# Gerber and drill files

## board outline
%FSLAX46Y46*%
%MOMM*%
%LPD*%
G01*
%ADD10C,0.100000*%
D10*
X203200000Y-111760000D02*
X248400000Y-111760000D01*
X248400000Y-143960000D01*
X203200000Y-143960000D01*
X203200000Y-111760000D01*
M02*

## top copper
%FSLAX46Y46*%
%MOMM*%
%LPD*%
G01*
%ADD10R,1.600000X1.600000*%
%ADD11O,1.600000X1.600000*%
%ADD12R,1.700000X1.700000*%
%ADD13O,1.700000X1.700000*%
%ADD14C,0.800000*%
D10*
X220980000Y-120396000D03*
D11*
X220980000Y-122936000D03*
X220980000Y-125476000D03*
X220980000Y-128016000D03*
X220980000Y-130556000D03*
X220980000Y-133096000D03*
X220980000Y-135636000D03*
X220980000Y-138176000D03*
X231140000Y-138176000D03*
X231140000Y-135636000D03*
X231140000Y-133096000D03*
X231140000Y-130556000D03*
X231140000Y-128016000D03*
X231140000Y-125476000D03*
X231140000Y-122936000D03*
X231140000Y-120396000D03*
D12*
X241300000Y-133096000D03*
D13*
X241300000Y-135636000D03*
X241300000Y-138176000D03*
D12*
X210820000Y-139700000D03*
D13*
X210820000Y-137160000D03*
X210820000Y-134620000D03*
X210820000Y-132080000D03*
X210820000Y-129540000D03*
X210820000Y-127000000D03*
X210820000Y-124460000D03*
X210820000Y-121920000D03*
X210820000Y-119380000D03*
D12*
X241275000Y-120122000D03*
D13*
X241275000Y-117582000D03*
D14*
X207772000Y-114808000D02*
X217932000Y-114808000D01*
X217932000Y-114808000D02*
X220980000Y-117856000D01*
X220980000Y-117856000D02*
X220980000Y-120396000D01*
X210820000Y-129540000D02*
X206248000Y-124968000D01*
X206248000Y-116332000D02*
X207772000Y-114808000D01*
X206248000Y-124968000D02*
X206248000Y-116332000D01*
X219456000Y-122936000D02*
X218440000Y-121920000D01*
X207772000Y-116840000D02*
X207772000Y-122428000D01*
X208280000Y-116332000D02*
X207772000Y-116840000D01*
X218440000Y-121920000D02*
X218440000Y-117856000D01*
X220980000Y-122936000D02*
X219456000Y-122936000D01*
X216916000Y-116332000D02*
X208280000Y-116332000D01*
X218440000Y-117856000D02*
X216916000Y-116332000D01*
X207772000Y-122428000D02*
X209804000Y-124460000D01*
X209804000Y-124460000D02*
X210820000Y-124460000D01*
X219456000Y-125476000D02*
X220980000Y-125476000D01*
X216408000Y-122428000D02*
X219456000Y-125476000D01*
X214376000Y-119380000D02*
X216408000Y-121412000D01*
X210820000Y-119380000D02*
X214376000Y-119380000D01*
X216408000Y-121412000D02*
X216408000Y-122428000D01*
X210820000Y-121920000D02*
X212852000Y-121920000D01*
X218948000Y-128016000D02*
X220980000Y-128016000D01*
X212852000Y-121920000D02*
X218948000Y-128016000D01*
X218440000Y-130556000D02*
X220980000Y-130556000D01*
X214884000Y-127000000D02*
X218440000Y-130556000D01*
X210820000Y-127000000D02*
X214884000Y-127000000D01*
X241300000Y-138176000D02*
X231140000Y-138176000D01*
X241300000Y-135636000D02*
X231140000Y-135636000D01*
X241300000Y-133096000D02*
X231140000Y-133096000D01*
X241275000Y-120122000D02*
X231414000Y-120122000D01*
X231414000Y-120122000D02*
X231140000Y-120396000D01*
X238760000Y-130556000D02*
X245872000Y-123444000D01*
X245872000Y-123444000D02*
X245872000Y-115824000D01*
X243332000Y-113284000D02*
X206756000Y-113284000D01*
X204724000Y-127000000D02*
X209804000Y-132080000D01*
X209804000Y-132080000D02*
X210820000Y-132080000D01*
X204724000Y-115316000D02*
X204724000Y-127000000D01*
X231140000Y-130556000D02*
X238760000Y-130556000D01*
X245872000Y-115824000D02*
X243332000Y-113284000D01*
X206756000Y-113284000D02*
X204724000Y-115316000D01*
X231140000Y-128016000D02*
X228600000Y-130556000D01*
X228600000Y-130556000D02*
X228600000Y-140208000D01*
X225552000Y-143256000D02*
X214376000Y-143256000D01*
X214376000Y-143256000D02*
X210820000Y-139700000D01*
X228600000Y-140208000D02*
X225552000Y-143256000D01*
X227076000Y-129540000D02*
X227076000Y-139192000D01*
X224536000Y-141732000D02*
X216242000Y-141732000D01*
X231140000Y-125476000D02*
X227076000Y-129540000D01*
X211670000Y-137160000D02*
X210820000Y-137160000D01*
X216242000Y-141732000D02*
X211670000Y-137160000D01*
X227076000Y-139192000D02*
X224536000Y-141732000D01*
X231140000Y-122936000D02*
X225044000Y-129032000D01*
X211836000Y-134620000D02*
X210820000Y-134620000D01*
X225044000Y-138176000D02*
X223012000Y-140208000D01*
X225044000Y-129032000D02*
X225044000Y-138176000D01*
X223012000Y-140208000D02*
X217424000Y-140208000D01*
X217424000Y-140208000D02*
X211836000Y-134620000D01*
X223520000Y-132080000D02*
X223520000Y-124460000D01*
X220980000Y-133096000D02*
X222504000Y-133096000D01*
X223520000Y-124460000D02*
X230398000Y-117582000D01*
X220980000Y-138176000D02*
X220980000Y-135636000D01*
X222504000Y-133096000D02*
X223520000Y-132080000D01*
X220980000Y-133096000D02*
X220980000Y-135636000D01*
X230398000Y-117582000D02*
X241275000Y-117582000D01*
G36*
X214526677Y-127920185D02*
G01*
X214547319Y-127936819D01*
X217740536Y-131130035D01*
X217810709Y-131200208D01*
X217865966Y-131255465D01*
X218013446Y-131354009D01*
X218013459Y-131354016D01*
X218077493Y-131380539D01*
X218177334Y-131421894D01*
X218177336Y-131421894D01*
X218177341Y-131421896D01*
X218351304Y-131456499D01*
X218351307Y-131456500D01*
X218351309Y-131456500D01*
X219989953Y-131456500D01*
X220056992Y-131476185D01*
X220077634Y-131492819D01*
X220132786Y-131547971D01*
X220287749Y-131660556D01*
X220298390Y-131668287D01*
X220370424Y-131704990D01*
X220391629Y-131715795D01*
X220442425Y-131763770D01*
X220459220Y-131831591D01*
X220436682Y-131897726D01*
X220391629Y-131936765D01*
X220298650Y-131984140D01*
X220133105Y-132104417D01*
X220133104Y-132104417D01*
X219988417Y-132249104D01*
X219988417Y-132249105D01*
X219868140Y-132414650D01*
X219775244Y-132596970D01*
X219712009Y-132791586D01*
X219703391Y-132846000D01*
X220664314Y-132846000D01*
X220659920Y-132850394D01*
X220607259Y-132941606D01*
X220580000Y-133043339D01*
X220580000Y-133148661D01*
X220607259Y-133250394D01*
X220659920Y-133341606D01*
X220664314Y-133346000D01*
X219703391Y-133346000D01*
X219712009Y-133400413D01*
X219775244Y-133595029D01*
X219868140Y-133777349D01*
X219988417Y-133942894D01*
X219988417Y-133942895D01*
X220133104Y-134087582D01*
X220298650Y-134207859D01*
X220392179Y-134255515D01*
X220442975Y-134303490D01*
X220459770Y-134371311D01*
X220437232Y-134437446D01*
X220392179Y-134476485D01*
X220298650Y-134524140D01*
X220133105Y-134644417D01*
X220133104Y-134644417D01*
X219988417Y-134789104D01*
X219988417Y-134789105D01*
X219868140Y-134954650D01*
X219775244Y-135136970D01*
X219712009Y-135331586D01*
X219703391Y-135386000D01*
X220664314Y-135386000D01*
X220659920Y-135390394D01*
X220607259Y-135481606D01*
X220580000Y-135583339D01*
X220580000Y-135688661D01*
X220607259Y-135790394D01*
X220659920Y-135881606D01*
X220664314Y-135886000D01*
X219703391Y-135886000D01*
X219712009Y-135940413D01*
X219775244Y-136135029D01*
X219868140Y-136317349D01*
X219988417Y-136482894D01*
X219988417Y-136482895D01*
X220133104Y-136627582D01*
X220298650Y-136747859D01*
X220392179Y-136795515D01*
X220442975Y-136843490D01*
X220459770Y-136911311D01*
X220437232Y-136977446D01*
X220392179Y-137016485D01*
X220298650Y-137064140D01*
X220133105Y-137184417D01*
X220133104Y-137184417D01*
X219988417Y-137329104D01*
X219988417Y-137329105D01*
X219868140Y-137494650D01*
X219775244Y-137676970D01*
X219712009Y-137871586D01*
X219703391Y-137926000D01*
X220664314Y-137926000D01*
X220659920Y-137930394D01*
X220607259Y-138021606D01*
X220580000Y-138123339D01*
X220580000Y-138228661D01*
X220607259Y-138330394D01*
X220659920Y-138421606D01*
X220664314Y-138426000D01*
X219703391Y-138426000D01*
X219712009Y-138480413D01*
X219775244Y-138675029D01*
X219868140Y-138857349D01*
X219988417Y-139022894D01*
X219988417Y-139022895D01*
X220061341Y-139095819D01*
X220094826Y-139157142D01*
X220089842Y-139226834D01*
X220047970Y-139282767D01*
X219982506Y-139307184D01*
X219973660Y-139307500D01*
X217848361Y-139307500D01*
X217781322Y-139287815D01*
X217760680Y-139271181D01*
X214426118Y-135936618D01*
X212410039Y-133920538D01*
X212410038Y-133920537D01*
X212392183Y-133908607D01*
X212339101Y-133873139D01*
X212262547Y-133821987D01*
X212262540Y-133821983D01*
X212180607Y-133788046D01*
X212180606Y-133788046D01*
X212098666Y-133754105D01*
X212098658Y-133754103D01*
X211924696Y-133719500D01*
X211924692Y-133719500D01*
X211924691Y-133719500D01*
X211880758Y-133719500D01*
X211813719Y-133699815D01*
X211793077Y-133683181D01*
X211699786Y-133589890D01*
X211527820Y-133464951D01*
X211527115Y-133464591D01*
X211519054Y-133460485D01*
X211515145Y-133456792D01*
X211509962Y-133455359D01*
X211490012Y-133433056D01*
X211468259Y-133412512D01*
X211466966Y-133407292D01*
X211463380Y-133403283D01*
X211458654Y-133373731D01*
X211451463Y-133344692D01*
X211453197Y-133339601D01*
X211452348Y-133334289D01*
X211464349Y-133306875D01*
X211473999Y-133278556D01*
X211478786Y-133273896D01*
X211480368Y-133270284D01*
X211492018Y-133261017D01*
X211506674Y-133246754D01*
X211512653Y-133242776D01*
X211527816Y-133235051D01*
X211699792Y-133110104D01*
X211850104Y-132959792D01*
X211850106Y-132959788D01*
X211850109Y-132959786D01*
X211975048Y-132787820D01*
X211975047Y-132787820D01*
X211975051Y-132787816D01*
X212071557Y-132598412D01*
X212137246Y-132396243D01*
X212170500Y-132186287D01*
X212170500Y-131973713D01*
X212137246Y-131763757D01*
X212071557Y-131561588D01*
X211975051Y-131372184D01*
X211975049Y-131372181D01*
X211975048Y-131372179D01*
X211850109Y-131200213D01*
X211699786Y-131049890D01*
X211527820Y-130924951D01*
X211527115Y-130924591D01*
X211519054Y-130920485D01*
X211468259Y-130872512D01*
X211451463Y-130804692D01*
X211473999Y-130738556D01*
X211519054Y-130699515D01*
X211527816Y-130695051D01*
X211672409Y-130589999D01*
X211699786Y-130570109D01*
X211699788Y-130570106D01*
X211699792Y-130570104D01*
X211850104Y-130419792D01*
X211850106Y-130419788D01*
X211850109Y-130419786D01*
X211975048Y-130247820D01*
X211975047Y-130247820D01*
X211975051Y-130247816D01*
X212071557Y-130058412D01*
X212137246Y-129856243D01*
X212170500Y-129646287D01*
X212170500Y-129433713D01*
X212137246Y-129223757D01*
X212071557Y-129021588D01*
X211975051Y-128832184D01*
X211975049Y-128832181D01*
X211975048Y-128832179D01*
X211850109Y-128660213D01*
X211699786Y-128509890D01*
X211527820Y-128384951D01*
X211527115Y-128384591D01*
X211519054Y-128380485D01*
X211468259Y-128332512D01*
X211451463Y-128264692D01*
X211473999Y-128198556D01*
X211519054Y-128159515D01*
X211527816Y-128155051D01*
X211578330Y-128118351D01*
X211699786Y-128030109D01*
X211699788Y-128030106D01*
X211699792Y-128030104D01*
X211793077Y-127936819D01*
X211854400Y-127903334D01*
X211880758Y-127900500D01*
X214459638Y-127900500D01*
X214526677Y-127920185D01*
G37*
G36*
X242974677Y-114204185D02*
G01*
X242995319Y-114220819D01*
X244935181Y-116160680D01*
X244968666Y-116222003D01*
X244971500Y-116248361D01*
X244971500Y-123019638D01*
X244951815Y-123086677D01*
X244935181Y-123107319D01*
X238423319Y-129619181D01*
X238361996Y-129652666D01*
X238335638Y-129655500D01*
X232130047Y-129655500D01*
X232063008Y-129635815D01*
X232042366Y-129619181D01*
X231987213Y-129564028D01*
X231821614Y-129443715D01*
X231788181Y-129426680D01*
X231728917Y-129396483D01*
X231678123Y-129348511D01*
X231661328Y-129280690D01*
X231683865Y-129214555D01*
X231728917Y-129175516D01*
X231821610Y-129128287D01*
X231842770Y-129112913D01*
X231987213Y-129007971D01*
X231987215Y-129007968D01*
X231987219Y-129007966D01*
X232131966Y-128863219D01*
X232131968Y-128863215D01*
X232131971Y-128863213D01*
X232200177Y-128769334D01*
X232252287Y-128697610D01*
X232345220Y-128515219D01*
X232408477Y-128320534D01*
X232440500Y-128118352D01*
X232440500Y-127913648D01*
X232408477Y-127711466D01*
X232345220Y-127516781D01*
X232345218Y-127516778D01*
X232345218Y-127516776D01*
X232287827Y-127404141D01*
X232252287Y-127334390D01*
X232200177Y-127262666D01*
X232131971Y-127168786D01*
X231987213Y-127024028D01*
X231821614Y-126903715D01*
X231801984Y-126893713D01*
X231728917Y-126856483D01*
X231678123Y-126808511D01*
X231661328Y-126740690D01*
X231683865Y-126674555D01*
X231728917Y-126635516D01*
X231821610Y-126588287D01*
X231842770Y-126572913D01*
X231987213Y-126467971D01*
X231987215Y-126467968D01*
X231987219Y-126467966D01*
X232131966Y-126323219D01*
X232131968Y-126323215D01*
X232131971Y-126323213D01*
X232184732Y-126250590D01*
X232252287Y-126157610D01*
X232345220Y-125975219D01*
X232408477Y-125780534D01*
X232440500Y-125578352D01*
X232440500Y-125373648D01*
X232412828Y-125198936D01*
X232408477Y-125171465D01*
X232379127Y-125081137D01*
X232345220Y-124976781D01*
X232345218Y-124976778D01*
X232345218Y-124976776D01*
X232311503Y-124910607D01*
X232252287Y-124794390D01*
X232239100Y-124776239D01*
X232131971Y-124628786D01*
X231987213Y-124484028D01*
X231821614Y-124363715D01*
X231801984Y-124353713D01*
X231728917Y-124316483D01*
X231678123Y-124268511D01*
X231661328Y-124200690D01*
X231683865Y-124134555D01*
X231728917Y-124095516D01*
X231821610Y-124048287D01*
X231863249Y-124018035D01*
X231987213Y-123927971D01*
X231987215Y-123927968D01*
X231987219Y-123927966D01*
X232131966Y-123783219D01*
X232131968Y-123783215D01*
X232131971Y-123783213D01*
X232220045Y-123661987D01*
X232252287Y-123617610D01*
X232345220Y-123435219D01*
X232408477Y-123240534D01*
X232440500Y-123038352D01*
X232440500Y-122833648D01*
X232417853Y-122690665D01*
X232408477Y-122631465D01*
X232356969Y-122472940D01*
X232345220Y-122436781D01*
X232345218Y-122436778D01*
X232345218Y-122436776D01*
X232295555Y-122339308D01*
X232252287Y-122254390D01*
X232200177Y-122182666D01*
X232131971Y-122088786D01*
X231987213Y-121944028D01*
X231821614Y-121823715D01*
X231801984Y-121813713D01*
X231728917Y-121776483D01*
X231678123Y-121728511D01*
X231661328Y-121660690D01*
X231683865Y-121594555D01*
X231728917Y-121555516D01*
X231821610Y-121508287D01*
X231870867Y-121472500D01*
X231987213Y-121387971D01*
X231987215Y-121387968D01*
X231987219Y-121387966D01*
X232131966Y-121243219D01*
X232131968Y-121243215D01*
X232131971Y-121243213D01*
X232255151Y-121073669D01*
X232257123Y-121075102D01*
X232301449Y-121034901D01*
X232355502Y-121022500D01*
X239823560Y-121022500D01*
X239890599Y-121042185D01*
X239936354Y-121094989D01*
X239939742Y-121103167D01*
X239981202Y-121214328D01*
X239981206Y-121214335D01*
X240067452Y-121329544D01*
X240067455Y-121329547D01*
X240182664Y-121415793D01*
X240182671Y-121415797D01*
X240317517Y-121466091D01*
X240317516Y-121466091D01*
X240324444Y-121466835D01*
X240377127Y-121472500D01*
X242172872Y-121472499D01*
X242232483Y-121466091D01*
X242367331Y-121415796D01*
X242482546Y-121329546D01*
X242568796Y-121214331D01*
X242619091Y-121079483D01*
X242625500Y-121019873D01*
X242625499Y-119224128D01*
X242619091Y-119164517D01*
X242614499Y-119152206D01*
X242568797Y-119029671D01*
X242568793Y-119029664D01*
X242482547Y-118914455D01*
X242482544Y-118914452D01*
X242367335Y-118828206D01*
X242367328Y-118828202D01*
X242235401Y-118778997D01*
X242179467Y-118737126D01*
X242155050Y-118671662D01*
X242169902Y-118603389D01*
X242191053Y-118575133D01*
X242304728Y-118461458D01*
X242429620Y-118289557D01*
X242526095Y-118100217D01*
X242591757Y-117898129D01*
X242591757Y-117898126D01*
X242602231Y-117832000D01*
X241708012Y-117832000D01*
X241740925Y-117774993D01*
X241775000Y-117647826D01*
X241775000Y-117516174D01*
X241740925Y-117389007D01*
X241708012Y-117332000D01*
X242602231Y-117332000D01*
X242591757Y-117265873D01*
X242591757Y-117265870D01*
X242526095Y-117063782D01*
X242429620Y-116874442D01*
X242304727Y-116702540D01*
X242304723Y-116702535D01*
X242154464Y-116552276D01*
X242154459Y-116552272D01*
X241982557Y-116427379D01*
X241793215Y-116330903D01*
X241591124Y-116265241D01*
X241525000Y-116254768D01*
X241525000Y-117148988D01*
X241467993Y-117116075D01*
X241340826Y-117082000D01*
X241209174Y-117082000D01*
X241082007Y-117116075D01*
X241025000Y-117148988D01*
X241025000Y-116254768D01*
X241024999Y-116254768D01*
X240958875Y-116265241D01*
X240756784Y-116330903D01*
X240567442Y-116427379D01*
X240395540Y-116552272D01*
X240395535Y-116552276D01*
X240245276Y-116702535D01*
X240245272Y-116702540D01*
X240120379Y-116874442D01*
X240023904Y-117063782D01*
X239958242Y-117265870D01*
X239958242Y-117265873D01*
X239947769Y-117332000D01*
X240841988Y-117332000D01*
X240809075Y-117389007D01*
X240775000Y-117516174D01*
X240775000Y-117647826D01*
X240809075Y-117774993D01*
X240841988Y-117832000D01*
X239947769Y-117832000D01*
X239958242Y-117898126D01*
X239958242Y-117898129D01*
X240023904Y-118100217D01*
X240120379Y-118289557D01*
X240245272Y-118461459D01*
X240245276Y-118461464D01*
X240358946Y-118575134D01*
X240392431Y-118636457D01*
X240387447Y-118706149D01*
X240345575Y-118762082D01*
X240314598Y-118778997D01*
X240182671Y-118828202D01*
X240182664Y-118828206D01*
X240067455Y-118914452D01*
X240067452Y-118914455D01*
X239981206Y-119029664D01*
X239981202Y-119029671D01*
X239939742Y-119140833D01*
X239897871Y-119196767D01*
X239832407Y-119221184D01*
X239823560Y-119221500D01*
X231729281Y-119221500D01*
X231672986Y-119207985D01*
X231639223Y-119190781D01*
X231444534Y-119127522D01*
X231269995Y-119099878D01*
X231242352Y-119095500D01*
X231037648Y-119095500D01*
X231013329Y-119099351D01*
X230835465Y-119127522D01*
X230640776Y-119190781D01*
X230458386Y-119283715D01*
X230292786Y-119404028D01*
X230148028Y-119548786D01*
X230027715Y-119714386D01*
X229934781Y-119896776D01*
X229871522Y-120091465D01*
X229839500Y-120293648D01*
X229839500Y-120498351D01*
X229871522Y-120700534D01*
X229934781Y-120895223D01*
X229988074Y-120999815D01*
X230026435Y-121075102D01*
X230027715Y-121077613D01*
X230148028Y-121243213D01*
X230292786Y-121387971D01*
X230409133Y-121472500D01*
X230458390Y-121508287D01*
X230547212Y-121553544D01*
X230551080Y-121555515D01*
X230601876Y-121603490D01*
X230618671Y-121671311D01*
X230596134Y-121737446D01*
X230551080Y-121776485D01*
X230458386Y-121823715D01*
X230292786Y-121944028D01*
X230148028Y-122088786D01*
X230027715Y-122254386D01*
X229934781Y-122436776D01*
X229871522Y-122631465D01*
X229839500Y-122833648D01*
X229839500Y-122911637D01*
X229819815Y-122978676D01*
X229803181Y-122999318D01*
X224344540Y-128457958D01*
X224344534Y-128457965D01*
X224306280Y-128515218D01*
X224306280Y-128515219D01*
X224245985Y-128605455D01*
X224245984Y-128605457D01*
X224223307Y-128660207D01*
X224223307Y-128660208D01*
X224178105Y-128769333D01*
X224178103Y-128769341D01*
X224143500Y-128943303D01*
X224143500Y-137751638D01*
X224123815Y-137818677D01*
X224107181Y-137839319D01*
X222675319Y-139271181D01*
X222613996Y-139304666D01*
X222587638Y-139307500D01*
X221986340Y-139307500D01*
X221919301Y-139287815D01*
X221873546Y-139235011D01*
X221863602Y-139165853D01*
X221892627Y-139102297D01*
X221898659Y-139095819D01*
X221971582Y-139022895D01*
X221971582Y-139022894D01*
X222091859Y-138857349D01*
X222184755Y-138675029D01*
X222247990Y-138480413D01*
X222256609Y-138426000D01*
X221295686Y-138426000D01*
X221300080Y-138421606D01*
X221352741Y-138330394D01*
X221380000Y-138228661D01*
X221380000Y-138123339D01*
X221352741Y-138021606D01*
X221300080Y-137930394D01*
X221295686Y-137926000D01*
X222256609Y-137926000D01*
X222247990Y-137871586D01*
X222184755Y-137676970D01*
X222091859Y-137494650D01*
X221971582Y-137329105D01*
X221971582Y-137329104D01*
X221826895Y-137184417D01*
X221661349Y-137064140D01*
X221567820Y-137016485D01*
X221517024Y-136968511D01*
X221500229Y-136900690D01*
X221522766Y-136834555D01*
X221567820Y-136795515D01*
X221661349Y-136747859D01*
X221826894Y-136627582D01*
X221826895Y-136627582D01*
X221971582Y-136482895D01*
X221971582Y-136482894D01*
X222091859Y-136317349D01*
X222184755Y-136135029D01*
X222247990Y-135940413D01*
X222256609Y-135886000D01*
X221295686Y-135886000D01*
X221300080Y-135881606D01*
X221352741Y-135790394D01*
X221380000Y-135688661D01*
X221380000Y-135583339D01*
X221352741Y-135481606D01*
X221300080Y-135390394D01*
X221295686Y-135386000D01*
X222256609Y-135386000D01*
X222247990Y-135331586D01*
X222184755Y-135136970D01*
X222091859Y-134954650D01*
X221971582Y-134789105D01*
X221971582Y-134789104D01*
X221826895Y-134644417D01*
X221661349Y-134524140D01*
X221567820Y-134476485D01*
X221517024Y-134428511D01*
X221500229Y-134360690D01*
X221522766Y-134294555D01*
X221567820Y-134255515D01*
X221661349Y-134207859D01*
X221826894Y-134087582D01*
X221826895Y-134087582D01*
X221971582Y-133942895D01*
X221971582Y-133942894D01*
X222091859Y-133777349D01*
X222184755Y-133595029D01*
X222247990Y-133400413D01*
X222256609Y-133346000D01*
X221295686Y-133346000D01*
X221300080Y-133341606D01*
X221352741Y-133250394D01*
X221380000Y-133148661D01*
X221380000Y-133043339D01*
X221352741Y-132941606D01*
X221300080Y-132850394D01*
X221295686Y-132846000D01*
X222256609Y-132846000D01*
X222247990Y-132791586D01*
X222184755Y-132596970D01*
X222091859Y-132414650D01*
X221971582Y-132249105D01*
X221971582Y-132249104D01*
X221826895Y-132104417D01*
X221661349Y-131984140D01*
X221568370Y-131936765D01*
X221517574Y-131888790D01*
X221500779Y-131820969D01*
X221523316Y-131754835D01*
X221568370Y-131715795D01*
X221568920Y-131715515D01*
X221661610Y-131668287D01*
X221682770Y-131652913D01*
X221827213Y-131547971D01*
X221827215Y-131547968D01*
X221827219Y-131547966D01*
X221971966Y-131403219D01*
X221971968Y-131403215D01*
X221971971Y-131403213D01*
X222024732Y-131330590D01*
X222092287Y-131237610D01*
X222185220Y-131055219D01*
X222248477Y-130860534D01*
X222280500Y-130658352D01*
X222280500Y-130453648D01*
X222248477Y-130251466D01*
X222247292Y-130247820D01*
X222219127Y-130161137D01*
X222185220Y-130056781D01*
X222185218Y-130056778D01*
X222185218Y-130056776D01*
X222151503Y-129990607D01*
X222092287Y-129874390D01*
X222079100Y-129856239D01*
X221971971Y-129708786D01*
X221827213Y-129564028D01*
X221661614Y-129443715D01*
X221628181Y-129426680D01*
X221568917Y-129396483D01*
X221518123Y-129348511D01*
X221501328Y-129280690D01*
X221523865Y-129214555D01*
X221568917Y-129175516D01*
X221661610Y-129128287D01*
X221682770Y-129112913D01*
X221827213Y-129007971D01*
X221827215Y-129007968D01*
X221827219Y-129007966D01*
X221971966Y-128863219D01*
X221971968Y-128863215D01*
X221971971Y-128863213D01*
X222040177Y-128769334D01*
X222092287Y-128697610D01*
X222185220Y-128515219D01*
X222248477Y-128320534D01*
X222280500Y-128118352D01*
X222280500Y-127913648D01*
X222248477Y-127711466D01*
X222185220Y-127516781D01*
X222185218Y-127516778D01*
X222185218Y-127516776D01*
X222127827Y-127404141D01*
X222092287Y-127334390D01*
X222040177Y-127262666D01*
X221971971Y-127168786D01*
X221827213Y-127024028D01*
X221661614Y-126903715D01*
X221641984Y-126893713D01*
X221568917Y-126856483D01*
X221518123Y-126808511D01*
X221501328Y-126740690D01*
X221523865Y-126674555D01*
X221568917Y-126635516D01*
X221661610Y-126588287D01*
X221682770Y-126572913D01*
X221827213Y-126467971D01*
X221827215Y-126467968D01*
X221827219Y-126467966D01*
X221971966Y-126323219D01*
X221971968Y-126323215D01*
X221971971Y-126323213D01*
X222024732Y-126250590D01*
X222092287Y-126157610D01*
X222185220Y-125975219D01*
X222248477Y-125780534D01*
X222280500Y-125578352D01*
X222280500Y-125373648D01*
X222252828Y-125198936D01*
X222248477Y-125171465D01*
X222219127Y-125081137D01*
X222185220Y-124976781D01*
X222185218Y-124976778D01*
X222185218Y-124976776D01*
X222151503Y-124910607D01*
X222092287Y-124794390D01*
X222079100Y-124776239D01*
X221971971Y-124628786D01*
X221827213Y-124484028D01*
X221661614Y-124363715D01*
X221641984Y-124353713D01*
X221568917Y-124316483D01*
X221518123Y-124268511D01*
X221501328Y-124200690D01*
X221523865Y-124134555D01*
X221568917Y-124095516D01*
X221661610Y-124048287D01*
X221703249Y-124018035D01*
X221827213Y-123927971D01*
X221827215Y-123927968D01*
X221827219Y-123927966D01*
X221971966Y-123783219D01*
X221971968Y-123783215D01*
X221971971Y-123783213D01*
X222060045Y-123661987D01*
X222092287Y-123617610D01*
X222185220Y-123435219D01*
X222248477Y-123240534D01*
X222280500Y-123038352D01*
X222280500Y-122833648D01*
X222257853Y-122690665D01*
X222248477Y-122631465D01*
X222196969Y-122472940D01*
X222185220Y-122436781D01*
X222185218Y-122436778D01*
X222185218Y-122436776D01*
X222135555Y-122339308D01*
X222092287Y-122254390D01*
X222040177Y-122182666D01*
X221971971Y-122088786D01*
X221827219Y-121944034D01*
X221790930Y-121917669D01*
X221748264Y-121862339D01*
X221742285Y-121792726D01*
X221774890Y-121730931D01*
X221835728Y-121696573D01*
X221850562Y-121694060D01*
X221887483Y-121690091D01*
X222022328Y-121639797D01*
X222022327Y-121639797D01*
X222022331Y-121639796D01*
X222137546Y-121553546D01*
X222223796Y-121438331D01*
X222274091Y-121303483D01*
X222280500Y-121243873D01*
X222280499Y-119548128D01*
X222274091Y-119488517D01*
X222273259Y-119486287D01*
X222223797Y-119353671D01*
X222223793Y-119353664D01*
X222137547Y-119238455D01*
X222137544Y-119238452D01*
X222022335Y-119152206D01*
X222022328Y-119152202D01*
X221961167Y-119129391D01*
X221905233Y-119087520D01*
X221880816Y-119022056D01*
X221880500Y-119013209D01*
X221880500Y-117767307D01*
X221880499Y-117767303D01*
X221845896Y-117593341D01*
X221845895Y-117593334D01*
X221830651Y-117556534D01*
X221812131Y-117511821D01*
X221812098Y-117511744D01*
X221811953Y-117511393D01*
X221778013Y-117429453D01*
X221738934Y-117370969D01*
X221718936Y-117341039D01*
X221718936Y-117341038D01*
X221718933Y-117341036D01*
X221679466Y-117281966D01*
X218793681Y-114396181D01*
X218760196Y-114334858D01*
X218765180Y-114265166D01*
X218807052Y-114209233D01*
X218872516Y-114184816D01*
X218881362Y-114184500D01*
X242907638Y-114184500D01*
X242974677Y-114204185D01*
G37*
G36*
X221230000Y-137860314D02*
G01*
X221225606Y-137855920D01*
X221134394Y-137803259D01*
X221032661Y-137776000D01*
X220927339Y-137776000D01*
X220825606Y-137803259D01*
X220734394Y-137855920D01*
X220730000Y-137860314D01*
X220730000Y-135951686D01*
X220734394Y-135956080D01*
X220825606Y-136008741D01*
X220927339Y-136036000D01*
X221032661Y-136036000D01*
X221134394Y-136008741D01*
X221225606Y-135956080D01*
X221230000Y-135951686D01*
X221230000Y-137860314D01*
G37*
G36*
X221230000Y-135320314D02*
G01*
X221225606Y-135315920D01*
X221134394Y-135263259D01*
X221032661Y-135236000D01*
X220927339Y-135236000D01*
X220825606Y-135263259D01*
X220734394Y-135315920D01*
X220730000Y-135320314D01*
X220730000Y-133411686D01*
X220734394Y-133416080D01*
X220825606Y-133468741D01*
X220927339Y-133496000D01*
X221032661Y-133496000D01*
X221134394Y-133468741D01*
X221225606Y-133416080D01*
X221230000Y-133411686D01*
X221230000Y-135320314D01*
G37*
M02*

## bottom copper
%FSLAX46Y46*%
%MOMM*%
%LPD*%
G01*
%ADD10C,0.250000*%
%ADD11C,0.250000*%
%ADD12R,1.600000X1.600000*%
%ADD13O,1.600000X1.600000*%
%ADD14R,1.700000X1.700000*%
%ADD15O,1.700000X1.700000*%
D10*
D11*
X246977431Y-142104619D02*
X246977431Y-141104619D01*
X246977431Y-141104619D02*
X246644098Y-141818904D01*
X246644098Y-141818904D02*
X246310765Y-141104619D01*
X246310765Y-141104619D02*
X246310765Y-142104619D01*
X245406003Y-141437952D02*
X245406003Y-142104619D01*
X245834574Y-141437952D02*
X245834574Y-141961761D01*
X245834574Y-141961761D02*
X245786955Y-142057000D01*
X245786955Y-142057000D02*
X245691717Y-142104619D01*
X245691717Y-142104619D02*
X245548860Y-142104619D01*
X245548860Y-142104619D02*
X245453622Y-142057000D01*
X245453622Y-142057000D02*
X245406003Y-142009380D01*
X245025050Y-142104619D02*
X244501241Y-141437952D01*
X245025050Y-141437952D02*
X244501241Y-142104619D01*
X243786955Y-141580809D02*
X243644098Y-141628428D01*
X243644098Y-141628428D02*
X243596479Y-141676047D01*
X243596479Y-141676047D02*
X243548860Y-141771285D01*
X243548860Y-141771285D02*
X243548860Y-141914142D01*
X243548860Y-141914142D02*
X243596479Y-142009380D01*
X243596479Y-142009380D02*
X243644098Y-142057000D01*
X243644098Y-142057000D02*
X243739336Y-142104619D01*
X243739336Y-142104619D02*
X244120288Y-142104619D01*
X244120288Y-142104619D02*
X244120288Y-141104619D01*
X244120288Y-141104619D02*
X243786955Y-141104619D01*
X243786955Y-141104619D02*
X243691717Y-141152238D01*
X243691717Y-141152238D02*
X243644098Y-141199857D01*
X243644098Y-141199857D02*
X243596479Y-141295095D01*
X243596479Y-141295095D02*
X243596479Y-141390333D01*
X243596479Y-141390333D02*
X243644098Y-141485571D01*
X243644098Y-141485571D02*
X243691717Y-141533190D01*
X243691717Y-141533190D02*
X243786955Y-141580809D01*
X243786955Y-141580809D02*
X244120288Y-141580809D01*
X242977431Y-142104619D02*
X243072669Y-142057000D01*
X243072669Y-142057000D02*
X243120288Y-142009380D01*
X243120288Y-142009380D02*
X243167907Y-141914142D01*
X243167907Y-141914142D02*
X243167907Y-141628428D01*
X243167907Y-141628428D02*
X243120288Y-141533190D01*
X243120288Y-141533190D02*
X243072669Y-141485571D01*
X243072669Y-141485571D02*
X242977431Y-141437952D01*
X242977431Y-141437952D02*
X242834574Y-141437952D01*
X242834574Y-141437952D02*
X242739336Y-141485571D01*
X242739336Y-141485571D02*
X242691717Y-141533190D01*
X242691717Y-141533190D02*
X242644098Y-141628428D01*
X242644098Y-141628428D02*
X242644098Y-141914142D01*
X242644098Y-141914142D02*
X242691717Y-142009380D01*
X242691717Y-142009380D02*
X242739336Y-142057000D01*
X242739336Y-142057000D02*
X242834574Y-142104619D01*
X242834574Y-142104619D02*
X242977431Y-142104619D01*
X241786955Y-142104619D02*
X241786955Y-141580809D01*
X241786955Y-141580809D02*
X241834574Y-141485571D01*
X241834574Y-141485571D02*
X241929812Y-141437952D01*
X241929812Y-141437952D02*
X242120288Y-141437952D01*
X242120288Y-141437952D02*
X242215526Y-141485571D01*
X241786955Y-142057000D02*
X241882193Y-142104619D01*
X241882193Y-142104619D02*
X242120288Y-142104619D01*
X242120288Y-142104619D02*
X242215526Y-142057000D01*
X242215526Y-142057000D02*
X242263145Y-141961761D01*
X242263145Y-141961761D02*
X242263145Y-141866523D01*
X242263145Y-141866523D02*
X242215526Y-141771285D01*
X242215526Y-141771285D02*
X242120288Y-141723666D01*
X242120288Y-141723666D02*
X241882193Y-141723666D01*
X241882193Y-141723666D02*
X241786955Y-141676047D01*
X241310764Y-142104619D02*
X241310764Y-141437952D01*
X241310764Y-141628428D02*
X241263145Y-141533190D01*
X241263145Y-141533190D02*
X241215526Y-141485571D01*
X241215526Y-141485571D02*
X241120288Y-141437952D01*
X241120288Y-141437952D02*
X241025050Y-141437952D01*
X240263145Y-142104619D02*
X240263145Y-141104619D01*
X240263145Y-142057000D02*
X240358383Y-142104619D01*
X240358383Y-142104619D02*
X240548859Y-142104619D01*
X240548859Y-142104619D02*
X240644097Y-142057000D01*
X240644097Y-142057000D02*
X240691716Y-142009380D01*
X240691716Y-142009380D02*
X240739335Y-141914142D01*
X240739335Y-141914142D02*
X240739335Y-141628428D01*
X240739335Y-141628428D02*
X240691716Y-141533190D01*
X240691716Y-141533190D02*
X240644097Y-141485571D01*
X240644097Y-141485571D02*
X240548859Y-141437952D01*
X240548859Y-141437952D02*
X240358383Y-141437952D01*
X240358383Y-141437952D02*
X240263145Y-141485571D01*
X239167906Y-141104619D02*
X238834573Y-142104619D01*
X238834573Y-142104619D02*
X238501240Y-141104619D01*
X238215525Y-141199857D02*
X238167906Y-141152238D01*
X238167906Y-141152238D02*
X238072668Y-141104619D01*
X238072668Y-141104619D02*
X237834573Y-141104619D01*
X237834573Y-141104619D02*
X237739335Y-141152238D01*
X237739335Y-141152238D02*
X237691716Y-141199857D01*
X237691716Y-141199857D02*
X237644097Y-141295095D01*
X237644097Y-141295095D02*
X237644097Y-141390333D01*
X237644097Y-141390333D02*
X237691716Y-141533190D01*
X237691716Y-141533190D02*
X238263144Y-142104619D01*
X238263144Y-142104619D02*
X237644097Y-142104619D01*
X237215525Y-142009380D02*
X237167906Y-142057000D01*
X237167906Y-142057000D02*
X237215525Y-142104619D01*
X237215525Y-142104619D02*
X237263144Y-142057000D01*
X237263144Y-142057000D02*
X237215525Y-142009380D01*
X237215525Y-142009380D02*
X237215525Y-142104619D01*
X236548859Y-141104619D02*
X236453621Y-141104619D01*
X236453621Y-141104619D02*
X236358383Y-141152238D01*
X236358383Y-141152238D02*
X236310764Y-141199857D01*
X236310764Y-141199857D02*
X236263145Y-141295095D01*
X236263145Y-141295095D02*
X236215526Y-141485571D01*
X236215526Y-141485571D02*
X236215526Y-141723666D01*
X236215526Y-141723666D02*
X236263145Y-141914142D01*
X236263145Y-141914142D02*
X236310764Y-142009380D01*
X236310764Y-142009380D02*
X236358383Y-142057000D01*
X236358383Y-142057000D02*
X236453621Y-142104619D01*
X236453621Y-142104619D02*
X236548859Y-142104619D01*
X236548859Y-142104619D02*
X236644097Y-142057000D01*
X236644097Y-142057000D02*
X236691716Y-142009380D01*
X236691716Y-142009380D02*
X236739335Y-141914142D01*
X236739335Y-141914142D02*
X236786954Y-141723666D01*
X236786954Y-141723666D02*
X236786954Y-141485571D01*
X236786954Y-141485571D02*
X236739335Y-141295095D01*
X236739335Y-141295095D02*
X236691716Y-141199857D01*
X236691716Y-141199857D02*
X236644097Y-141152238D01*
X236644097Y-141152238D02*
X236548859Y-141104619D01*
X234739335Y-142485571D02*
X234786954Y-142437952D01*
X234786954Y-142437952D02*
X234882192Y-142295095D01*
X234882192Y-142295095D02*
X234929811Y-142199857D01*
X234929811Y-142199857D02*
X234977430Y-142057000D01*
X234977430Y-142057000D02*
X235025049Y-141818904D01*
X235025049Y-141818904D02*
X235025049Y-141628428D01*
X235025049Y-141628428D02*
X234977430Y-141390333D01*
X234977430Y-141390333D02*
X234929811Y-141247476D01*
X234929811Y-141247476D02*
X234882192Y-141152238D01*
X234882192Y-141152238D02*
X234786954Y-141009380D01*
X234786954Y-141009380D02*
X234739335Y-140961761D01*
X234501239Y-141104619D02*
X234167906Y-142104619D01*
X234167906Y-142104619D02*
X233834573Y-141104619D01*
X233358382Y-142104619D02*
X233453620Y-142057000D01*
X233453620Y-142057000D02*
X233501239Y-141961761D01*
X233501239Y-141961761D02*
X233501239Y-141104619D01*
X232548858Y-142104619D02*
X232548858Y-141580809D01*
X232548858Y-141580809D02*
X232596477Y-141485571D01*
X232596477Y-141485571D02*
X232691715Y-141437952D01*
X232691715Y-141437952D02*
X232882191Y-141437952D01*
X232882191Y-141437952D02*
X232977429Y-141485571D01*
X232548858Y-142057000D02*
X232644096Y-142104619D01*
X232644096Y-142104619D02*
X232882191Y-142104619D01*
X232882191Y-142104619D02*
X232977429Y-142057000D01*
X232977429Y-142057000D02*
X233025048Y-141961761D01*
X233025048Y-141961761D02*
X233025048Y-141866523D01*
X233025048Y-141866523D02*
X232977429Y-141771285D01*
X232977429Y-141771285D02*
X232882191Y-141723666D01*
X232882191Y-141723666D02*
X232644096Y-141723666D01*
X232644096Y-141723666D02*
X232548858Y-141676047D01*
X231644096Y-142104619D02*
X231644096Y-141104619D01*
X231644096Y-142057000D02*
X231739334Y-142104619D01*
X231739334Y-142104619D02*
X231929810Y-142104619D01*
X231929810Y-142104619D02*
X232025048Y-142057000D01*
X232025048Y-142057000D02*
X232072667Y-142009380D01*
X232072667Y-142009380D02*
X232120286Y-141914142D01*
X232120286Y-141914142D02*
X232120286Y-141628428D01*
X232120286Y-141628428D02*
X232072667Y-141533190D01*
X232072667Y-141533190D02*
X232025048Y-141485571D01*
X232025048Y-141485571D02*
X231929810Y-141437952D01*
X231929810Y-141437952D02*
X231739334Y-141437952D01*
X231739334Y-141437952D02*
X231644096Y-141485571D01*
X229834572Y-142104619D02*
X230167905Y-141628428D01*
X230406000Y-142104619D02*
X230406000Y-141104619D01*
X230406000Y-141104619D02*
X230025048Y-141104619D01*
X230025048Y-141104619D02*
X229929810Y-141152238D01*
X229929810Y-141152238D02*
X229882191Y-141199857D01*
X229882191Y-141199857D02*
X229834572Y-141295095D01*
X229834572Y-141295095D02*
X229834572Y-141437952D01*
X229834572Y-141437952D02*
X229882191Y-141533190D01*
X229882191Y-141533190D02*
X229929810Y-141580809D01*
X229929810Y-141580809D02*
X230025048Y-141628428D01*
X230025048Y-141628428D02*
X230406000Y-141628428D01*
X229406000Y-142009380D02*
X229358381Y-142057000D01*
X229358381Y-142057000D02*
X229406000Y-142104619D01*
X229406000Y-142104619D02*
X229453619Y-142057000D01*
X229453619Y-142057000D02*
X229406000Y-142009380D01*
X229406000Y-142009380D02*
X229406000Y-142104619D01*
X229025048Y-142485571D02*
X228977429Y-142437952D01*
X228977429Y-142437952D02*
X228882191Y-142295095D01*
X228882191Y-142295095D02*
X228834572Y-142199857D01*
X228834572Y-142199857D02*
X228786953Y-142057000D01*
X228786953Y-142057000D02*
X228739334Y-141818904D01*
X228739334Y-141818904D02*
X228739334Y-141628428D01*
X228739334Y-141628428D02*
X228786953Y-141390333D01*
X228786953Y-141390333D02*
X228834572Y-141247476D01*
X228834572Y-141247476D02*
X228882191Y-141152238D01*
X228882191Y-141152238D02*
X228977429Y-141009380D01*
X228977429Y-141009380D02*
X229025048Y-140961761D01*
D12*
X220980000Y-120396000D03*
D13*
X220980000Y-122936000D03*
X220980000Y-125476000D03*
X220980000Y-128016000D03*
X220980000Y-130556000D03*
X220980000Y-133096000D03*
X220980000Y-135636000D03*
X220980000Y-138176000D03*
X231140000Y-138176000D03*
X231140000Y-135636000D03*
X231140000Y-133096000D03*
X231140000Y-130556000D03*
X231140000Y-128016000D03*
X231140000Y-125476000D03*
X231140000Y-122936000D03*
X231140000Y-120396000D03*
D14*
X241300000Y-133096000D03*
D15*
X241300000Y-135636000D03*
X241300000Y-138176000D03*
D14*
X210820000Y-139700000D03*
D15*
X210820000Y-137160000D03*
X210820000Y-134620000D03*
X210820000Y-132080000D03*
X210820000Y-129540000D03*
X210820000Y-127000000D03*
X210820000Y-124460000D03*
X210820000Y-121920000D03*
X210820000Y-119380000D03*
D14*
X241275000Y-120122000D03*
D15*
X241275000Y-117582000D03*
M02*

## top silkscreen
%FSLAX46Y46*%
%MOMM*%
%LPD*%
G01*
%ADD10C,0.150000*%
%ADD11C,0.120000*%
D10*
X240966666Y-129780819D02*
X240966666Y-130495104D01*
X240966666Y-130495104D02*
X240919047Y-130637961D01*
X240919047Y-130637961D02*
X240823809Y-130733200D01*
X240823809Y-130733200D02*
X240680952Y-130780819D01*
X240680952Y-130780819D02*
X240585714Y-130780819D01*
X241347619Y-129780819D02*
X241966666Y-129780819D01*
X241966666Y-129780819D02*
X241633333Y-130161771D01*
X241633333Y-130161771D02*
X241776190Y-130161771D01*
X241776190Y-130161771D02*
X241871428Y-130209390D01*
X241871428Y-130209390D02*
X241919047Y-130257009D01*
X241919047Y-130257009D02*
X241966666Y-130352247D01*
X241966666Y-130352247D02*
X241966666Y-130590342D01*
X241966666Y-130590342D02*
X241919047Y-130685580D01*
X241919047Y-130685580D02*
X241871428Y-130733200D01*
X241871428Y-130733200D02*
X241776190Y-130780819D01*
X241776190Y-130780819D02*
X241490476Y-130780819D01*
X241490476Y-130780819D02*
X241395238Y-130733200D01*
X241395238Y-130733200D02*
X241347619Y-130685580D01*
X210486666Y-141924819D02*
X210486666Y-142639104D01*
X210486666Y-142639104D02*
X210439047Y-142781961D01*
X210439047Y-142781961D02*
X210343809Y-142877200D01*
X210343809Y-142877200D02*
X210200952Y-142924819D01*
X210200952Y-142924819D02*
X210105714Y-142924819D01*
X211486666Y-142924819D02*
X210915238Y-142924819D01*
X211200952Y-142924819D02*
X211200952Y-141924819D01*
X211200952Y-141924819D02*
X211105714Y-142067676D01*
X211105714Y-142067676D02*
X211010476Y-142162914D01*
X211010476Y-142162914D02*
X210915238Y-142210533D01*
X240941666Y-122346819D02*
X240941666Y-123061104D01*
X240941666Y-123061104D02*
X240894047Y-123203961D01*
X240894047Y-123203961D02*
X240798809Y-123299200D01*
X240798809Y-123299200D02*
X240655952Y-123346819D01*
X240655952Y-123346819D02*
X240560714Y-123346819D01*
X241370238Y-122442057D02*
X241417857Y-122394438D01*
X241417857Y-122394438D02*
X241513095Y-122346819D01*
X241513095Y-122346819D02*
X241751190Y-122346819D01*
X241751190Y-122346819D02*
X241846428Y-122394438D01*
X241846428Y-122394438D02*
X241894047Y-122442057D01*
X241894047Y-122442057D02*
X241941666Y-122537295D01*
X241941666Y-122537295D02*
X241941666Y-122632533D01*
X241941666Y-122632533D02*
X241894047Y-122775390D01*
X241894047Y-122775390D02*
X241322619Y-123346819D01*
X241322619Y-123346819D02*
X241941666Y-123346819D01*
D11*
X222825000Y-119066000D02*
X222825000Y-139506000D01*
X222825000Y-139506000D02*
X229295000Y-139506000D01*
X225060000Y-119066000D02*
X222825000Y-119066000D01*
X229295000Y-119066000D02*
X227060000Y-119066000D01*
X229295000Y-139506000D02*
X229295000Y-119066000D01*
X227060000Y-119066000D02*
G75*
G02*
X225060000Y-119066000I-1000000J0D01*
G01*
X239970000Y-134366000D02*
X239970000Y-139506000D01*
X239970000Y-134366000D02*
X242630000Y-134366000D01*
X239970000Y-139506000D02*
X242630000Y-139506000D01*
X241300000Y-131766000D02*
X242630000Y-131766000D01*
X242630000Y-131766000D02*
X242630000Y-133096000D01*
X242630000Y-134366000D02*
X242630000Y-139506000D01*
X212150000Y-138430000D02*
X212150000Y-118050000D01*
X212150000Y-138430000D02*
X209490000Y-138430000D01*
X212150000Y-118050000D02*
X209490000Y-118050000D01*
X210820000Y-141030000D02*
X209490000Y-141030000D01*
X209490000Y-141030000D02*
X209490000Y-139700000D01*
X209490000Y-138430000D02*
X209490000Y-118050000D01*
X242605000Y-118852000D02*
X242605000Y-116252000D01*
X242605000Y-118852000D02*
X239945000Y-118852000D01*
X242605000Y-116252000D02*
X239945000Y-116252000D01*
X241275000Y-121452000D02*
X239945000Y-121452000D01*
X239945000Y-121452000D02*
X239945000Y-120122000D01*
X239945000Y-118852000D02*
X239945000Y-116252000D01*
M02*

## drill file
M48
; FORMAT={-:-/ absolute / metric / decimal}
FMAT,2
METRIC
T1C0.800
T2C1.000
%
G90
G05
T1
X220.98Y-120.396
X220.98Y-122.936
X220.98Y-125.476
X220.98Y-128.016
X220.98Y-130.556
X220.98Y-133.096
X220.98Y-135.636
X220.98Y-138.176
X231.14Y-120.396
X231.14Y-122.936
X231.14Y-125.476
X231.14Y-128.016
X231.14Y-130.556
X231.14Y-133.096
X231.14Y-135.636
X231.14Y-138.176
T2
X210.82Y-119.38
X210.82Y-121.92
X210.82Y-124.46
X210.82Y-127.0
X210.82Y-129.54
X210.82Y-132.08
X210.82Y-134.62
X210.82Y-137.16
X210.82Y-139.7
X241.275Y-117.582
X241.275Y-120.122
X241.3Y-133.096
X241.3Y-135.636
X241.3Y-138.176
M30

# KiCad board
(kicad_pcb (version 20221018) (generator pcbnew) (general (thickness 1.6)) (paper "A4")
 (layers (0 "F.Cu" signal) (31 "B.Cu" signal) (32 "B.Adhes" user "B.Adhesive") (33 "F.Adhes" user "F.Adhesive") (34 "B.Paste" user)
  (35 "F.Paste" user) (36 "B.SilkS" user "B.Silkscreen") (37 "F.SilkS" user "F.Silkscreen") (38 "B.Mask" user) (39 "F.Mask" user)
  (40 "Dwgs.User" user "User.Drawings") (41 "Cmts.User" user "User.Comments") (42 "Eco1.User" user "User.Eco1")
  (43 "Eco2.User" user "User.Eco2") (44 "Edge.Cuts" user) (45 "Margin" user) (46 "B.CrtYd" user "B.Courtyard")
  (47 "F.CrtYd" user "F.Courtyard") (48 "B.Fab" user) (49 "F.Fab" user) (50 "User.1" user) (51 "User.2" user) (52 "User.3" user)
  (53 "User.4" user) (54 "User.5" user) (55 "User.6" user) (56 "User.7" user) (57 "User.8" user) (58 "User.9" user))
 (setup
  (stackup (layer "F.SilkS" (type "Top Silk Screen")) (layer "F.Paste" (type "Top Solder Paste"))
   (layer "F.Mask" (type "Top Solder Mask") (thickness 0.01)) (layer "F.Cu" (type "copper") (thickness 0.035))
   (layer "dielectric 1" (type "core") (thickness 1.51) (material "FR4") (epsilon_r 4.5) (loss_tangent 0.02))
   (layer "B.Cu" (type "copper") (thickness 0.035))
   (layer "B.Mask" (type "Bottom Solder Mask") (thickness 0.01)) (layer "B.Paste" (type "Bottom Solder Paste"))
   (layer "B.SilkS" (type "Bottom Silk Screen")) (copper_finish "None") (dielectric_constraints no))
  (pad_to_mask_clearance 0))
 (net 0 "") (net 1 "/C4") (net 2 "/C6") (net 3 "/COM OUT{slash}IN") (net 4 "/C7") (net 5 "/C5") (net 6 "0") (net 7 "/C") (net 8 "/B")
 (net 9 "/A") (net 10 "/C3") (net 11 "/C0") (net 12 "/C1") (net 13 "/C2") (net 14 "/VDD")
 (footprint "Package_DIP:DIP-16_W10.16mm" (layer "F.Cu") (at 220.98 120.396)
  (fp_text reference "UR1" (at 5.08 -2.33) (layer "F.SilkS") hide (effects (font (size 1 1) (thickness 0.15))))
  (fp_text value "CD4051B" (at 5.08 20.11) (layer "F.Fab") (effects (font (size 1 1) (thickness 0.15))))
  (fp_line (start 1.845 -1.33) (end 1.845 19.11) (stroke (width 0.12) (type solid)) (layer "F.SilkS"))
  (fp_line (start 1.845 19.11) (end 8.315 19.11) (stroke (width 0.12) (type solid)) (layer "F.SilkS"))
  (fp_line (start 4.08 -1.33) (end 1.845 -1.33) (stroke (width 0.12) (type solid)) (layer "F.SilkS"))
  (fp_line (start 8.315 -1.33) (end 6.08 -1.33) (stroke (width 0.12) (type solid)) (layer "F.SilkS"))
  (fp_line (start 8.315 19.11) (end 8.315 -1.33) (stroke (width 0.12) (type solid)) (layer "F.SilkS"))
  (fp_arc (start 6.08 -1.33) (mid 5.08 -0.33) (end 4.08 -1.33) (stroke (width 0.12) (type solid)) (layer "F.SilkS"))
  (pad "1" thru_hole rect (at 0 0) (size 1.6 1.6) (drill 0.8) (layers "*.Cu" "*.Mask") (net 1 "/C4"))
  (pad "2" thru_hole oval (at 0 2.54) (size 1.6 1.6) (drill 0.8) (layers "*.Cu" "*.Mask") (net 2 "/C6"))
  (pad "3" thru_hole oval (at 0 5.08) (size 1.6 1.6) (drill 0.8) (layers "*.Cu" "*.Mask") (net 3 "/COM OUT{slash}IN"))
  (pad "4" thru_hole oval (at 0 7.62) (size 1.6 1.6) (drill 0.8) (layers "*.Cu" "*.Mask") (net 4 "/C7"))
  (pad "5" thru_hole oval (at 0 10.16) (size 1.6 1.6) (drill 0.8) (layers "*.Cu" "*.Mask") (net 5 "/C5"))
  (pad "6" thru_hole oval (at 0 12.7) (size 1.6 1.6) (drill 0.8) (layers "*.Cu" "*.Mask") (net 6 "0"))
  (pad "7" thru_hole oval (at 0 15.24) (size 1.6 1.6) (drill 0.8) (layers "*.Cu" "*.Mask") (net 6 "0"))
  (pad "8" thru_hole oval (at 0 17.78) (size 1.6 1.6) (drill 0.8) (layers "*.Cu" "*.Mask") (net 6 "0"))
  (pad "9" thru_hole oval (at 10.16 17.78) (size 1.6 1.6) (drill 0.8) (layers "*.Cu" "*.Mask") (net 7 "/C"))
  (pad "10" thru_hole oval (at 10.16 15.24) (size 1.6 1.6) (drill 0.8) (layers "*.Cu" "*.Mask") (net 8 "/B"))
  (pad "11" thru_hole oval (at 10.16 12.7) (size 1.6 1.6) (drill 0.8) (layers "*.Cu" "*.Mask") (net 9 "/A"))
  (pad "12" thru_hole oval (at 10.16 10.16) (size 1.6 1.6) (drill 0.8) (layers "*.Cu" "*.Mask") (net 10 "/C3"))
  (pad "13" thru_hole oval (at 10.16 7.62) (size 1.6 1.6) (drill 0.8) (layers "*.Cu" "*.Mask") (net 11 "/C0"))
  (pad "14" thru_hole oval (at 10.16 5.08) (size 1.6 1.6) (drill 0.8) (layers "*.Cu" "*.Mask") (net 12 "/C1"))
  (pad "15" thru_hole oval (at 10.16 2.54) (size 1.6 1.6) (drill 0.8) (layers "*.Cu" "*.Mask") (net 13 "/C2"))
  (pad "16" thru_hole oval (at 10.16 0) (size 1.6 1.6) (drill 0.8) (layers "*.Cu" "*.Mask") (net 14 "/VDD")))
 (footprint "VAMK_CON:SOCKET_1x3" (layer "F.Cu") (at 241.3 133.096)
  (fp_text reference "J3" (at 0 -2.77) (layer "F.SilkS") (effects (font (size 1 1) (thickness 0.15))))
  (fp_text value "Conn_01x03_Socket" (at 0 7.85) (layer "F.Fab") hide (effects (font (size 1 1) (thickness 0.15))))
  (fp_line (start -1.33 1.27) (end -1.33 6.41) (stroke (width 0.12) (type solid)) (layer "F.SilkS"))
  (fp_line (start -1.33 1.27) (end 1.33 1.27) (stroke (width 0.12) (type solid)) (layer "F.SilkS"))
  (fp_line (start -1.33 6.41) (end 1.33 6.41) (stroke (width 0.12) (type solid)) (layer "F.SilkS"))
  (fp_line (start 0 -1.33) (end 1.33 -1.33) (stroke (width 0.12) (type solid)) (layer "F.SilkS"))
  (fp_line (start 1.33 -1.33) (end 1.33 0) (stroke (width 0.12) (type solid)) (layer "F.SilkS"))
  (fp_line (start 1.33 1.27) (end 1.33 6.41) (stroke (width 0.12) (type solid)) (layer "F.SilkS"))
  (pad "1" thru_hole rect (at 0 0) (size 1.7 1.7) (drill 1) (layers "*.Cu" "*.Mask") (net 9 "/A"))
  (pad "2" thru_hole oval (at 0 2.54) (size 1.7 1.7) (drill 1) (layers "*.Cu" "*.Mask") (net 8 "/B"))
  (pad "3" thru_hole oval (at 0 5.08) (size 1.7 1.7) (drill 1) (layers "*.Cu" "*.Mask") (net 7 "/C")))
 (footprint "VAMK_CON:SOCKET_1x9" (layer "F.Cu") (at 210.82 139.7 180)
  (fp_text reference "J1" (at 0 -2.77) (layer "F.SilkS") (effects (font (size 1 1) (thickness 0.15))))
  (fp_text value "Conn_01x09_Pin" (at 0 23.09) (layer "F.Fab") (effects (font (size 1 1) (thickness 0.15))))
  (fp_line (start -1.33 1.27) (end -1.33 21.65) (stroke (width 0.12) (type solid)) (layer "F.SilkS"))
  (fp_line (start -1.33 1.27) (end 1.33 1.27) (stroke (width 0.12) (type solid)) (layer "F.SilkS"))
  (fp_line (start -1.33 21.65) (end 1.33 21.65) (stroke (width 0.12) (type solid)) (layer "F.SilkS"))
  (fp_line (start 0 -1.33) (end 1.33 -1.33) (stroke (width 0.12) (type solid)) (layer "F.SilkS"))
  (fp_line (start 1.33 -1.33) (end 1.33 0) (stroke (width 0.12) (type solid)) (layer "F.SilkS"))
  (fp_line (start 1.33 1.27) (end 1.33 21.65) (stroke (width 0.12) (type solid)) (layer "F.SilkS"))
  (pad "1" thru_hole rect (at 0 0 180) (size 1.7 1.7) (drill 1) (layers "*.Cu" "*.Mask") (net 11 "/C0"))
  (pad "2" thru_hole oval (at 0 2.54 180) (size 1.7 1.7) (drill 1) (layers "*.Cu" "*.Mask") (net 12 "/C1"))
  (pad "3" thru_hole oval (at 0 5.08 180) (size 1.7 1.7) (drill 1) (layers "*.Cu" "*.Mask") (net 13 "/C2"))
  (pad "4" thru_hole oval (at 0 7.62 180) (size 1.7 1.7) (drill 1) (layers "*.Cu" "*.Mask") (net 10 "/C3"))
  (pad "5" thru_hole oval (at 0 10.16 180) (size 1.7 1.7) (drill 1) (layers "*.Cu" "*.Mask") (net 1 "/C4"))
  (pad "6" thru_hole oval (at 0 12.7 180) (size 1.7 1.7) (drill 1) (layers "*.Cu" "*.Mask") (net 5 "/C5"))
  (pad "7" thru_hole oval (at 0 15.24 180) (size 1.7 1.7) (drill 1) (layers "*.Cu" "*.Mask") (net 2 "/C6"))
  (pad "8" thru_hole oval (at 0 17.78 180) (size 1.7 1.7) (drill 1) (layers "*.Cu" "*.Mask") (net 4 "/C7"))
  (pad "9" thru_hole oval (at 0 20.32 180) (size 1.7 1.7) (drill 1) (layers "*.Cu" "*.Mask") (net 3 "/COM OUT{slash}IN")))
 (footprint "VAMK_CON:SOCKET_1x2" (layer "F.Cu") (at 241.275 120.122 180)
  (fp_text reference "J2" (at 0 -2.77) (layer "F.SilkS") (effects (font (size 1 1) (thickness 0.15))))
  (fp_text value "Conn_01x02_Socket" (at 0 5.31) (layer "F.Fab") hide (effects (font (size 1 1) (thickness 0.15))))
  (fp_line (start -1.33 1.27) (end -1.33 3.87) (stroke (width 0.12) (type solid)) (layer "F.SilkS"))
  (fp_line (start -1.33 1.27) (end 1.33 1.27) (stroke (width 0.12) (type solid)) (layer "F.SilkS"))
  (fp_line (start -1.33 3.87) (end 1.33 3.87) (stroke (width 0.12) (type solid)) (layer "F.SilkS"))
  (fp_line (start 0 -1.33) (end 1.33 -1.33) (stroke (width 0.12) (type solid)) (layer "F.SilkS"))
  (fp_line (start 1.33 -1.33) (end 1.33 0) (stroke (width 0.12) (type solid)) (layer "F.SilkS"))
  (fp_line (start 1.33 1.27) (end 1.33 3.87) (stroke (width 0.12) (type solid)) (layer "F.SilkS"))
  (pad "1" thru_hole rect (at 0 0 180) (size 1.7 1.7) (drill 1) (layers "*.Cu" "*.Mask") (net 14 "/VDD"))
  (pad "2" thru_hole oval (at 0 2.54 180) (size 1.7 1.7) (drill 1) (layers "*.Cu" "*.Mask") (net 6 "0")))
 (gr_rect (start 203.2 111.76) (end 248.4 143.96) (stroke (width 0.1) (type default)) (fill none) (layer "Edge.Cuts"))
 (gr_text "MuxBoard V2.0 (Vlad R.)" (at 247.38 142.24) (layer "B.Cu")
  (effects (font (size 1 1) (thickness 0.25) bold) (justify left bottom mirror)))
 (segment (start 207.772 114.808) (end 217.932 114.808) (width 0.8) (layer "F.Cu") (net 1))
 (segment (start 217.932 114.808) (end 220.98 117.856) (width 0.8) (layer "F.Cu") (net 1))
 (segment (start 220.98 117.856) (end 220.98 120.396) (width 0.8) (layer "F.Cu") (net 1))
 (segment (start 210.82 129.54) (end 206.248 124.968) (width 0.8) (layer "F.Cu") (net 1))
 (segment (start 206.248 116.332) (end 207.772 114.808) (width 0.8) (layer "F.Cu") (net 1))
 (segment (start 206.248 124.968) (end 206.248 116.332) (width 0.8) (layer "F.Cu") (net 1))
 (segment (start 219.456 122.936) (end 218.44 121.92) (width 0.8) (layer "F.Cu") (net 2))
 (segment (start 207.772 116.84) (end 207.772 122.428) (width 0.8) (layer "F.Cu") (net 2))
 (segment (start 208.28 116.332) (end 207.772 116.84) (width 0.8) (layer "F.Cu") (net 2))
 (segment (start 218.44 121.92) (end 218.44 117.856) (width 0.8) (layer "F.Cu") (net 2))
 (segment (start 220.98 122.936) (end 219.456 122.936) (width 0.8) (layer "F.Cu") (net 2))
 (segment (start 216.916 116.332) (end 208.28 116.332) (width 0.8) (layer "F.Cu") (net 2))
 (segment (start 218.44 117.856) (end 216.916 116.332) (width 0.8) (layer "F.Cu") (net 2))
 (segment (start 207.772 122.428) (end 209.804 124.46) (width 0.8) (layer "F.Cu") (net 2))
 (segment (start 209.804 124.46) (end 210.82 124.46) (width 0.8) (layer "F.Cu") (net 2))
 (segment (start 219.456 125.476) (end 220.98 125.476) (width 0.8) (layer "F.Cu") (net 3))
 (segment (start 216.408 122.428) (end 219.456 125.476) (width 0.8) (layer "F.Cu") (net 3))
 (segment (start 214.376 119.38) (end 216.408 121.412) (width 0.8) (layer "F.Cu") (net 3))
 (segment (start 210.82 119.38) (end 214.376 119.38) (width 0.8) (layer "F.Cu") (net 3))
 (segment (start 216.408 121.412) (end 216.408 122.428) (width 0.8) (layer "F.Cu") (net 3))
 (segment (start 210.82 121.92) (end 212.852 121.92) (width 0.8) (layer "F.Cu") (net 4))
 (segment (start 218.948 128.016) (end 220.98 128.016) (width 0.8) (layer "F.Cu") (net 4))
 (segment (start 212.852 121.92) (end 218.948 128.016) (width 0.8) (layer "F.Cu") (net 4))
 (segment (start 218.44 130.556) (end 220.98 130.556) (width 0.8) (layer "F.Cu") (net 5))
 (segment (start 214.884 127) (end 218.44 130.556) (width 0.8) (layer "F.Cu") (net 5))
 (segment (start 210.82 127) (end 214.884 127) (width 0.8) (layer "F.Cu") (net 5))
 (segment (start 241.3 138.176) (end 231.14 138.176) (width 0.8) (layer "F.Cu") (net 7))
 (segment (start 241.3 135.636) (end 231.14 135.636) (width 0.8) (layer "F.Cu") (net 8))
 (segment (start 241.3 133.096) (end 231.14 133.096) (width 0.8) (layer "F.Cu") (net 9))
 (segment (start 241.275 120.122) (end 231.414 120.122) (width 0.8) (layer "F.Cu") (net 14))
 (segment (start 231.414 120.122) (end 231.14 120.396) (width 0.8) (layer "F.Cu") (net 14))
 (segment (start 238.76 130.556) (end 245.872 123.444) (width 0.8) (layer "F.Cu") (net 10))
 (segment (start 245.872 123.444) (end 245.872 115.824) (width 0.8) (layer "F.Cu") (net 10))
 (segment (start 243.332 113.284) (end 206.756 113.284) (width 0.8) (layer "F.Cu") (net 10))
 (segment (start 204.724 127) (end 209.804 132.08) (width 0.8) (layer "F.Cu") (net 10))
 (segment (start 209.804 132.08) (end 210.82 132.08) (width 0.8) (layer "F.Cu") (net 10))
 (segment (start 204.724 115.316) (end 204.724 127) (width 0.8) (layer "F.Cu") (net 10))
 (segment (start 231.14 130.556) (end 238.76 130.556) (width 0.8) (layer "F.Cu") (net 10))
 (segment (start 245.872 115.824) (end 243.332 113.284) (width 0.8) (layer "F.Cu") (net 10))
 (segment (start 206.756 113.284) (end 204.724 115.316) (width 0.8) (layer "F.Cu") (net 10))
 (segment (start 231.14 128.016) (end 228.6 130.556) (width 0.8) (layer "F.Cu") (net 11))
 (segment (start 228.6 130.556) (end 228.6 140.208) (width 0.8) (layer "F.Cu") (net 11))
 (segment (start 225.552 143.256) (end 214.376 143.256) (width 0.8) (layer "F.Cu") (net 11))
 (segment (start 214.376 143.256) (end 210.82 139.7) (width 0.8) (layer "F.Cu") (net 11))
 (segment (start 228.6 140.208) (end 225.552 143.256) (width 0.8) (layer "F.Cu") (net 11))
 (segment (start 227.076 129.54) (end 227.076 139.192) (width 0.8) (layer "F.Cu") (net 12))
 (segment (start 224.536 141.732) (end 216.242 141.732) (width 0.8) (layer "F.Cu") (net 12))
 (segment (start 231.14 125.476) (end 227.076 129.54) (width 0.8) (layer "F.Cu") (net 12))
 (segment (start 211.67 137.16) (end 210.82 137.16) (width 0.8) (layer "F.Cu") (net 12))
 (segment (start 216.242 141.732) (end 211.67 137.16) (width 0.8) (layer "F.Cu") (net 12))
 (segment (start 227.076 139.192) (end 224.536 141.732) (width 0.8) (layer "F.Cu") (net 12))
 (segment (start 231.14 122.936) (end 225.044 129.032) (width 0.8) (layer "F.Cu") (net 13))
 (segment (start 211.836 134.62) (end 210.82 134.62) (width 0.8) (layer "F.Cu") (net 13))
 (segment (start 225.044 138.176) (end 223.012 140.208) (width 0.8) (layer "F.Cu") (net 13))
 (segment (start 225.044 129.032) (end 225.044 138.176) (width 0.8) (layer "F.Cu") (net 13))
 (segment (start 223.012 140.208) (end 217.424 140.208) (width 0.8) (layer "F.Cu") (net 13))
 (segment (start 217.424 140.208) (end 211.836 134.62) (width 0.8) (layer "F.Cu") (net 13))
 (segment (start 223.52 132.08) (end 223.52 124.46) (width 0.8) (layer "F.Cu") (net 6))
 (segment (start 220.98 133.096) (end 222.504 133.096) (width 0.8) (layer "F.Cu") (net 6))
 (segment (start 223.52 124.46) (end 230.398 117.582) (width 0.8) (layer "F.Cu") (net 6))
 (segment (start 220.98 138.176) (end 220.98 135.636) (width 0.8) (layer "F.Cu") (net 6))
 (segment (start 222.504 133.096) (end 223.52 132.08) (width 0.8) (layer "F.Cu") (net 6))
 (segment (start 220.98 133.096) (end 220.98 135.636) (width 0.8) (layer "F.Cu") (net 6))
 (segment (start 230.398 117.582) (end 241.275 117.582) (width 0.8) (layer "F.Cu") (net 6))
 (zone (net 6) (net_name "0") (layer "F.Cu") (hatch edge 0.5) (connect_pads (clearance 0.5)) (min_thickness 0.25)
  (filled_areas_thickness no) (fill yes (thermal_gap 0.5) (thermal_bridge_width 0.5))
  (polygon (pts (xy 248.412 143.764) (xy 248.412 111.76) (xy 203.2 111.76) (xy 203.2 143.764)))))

